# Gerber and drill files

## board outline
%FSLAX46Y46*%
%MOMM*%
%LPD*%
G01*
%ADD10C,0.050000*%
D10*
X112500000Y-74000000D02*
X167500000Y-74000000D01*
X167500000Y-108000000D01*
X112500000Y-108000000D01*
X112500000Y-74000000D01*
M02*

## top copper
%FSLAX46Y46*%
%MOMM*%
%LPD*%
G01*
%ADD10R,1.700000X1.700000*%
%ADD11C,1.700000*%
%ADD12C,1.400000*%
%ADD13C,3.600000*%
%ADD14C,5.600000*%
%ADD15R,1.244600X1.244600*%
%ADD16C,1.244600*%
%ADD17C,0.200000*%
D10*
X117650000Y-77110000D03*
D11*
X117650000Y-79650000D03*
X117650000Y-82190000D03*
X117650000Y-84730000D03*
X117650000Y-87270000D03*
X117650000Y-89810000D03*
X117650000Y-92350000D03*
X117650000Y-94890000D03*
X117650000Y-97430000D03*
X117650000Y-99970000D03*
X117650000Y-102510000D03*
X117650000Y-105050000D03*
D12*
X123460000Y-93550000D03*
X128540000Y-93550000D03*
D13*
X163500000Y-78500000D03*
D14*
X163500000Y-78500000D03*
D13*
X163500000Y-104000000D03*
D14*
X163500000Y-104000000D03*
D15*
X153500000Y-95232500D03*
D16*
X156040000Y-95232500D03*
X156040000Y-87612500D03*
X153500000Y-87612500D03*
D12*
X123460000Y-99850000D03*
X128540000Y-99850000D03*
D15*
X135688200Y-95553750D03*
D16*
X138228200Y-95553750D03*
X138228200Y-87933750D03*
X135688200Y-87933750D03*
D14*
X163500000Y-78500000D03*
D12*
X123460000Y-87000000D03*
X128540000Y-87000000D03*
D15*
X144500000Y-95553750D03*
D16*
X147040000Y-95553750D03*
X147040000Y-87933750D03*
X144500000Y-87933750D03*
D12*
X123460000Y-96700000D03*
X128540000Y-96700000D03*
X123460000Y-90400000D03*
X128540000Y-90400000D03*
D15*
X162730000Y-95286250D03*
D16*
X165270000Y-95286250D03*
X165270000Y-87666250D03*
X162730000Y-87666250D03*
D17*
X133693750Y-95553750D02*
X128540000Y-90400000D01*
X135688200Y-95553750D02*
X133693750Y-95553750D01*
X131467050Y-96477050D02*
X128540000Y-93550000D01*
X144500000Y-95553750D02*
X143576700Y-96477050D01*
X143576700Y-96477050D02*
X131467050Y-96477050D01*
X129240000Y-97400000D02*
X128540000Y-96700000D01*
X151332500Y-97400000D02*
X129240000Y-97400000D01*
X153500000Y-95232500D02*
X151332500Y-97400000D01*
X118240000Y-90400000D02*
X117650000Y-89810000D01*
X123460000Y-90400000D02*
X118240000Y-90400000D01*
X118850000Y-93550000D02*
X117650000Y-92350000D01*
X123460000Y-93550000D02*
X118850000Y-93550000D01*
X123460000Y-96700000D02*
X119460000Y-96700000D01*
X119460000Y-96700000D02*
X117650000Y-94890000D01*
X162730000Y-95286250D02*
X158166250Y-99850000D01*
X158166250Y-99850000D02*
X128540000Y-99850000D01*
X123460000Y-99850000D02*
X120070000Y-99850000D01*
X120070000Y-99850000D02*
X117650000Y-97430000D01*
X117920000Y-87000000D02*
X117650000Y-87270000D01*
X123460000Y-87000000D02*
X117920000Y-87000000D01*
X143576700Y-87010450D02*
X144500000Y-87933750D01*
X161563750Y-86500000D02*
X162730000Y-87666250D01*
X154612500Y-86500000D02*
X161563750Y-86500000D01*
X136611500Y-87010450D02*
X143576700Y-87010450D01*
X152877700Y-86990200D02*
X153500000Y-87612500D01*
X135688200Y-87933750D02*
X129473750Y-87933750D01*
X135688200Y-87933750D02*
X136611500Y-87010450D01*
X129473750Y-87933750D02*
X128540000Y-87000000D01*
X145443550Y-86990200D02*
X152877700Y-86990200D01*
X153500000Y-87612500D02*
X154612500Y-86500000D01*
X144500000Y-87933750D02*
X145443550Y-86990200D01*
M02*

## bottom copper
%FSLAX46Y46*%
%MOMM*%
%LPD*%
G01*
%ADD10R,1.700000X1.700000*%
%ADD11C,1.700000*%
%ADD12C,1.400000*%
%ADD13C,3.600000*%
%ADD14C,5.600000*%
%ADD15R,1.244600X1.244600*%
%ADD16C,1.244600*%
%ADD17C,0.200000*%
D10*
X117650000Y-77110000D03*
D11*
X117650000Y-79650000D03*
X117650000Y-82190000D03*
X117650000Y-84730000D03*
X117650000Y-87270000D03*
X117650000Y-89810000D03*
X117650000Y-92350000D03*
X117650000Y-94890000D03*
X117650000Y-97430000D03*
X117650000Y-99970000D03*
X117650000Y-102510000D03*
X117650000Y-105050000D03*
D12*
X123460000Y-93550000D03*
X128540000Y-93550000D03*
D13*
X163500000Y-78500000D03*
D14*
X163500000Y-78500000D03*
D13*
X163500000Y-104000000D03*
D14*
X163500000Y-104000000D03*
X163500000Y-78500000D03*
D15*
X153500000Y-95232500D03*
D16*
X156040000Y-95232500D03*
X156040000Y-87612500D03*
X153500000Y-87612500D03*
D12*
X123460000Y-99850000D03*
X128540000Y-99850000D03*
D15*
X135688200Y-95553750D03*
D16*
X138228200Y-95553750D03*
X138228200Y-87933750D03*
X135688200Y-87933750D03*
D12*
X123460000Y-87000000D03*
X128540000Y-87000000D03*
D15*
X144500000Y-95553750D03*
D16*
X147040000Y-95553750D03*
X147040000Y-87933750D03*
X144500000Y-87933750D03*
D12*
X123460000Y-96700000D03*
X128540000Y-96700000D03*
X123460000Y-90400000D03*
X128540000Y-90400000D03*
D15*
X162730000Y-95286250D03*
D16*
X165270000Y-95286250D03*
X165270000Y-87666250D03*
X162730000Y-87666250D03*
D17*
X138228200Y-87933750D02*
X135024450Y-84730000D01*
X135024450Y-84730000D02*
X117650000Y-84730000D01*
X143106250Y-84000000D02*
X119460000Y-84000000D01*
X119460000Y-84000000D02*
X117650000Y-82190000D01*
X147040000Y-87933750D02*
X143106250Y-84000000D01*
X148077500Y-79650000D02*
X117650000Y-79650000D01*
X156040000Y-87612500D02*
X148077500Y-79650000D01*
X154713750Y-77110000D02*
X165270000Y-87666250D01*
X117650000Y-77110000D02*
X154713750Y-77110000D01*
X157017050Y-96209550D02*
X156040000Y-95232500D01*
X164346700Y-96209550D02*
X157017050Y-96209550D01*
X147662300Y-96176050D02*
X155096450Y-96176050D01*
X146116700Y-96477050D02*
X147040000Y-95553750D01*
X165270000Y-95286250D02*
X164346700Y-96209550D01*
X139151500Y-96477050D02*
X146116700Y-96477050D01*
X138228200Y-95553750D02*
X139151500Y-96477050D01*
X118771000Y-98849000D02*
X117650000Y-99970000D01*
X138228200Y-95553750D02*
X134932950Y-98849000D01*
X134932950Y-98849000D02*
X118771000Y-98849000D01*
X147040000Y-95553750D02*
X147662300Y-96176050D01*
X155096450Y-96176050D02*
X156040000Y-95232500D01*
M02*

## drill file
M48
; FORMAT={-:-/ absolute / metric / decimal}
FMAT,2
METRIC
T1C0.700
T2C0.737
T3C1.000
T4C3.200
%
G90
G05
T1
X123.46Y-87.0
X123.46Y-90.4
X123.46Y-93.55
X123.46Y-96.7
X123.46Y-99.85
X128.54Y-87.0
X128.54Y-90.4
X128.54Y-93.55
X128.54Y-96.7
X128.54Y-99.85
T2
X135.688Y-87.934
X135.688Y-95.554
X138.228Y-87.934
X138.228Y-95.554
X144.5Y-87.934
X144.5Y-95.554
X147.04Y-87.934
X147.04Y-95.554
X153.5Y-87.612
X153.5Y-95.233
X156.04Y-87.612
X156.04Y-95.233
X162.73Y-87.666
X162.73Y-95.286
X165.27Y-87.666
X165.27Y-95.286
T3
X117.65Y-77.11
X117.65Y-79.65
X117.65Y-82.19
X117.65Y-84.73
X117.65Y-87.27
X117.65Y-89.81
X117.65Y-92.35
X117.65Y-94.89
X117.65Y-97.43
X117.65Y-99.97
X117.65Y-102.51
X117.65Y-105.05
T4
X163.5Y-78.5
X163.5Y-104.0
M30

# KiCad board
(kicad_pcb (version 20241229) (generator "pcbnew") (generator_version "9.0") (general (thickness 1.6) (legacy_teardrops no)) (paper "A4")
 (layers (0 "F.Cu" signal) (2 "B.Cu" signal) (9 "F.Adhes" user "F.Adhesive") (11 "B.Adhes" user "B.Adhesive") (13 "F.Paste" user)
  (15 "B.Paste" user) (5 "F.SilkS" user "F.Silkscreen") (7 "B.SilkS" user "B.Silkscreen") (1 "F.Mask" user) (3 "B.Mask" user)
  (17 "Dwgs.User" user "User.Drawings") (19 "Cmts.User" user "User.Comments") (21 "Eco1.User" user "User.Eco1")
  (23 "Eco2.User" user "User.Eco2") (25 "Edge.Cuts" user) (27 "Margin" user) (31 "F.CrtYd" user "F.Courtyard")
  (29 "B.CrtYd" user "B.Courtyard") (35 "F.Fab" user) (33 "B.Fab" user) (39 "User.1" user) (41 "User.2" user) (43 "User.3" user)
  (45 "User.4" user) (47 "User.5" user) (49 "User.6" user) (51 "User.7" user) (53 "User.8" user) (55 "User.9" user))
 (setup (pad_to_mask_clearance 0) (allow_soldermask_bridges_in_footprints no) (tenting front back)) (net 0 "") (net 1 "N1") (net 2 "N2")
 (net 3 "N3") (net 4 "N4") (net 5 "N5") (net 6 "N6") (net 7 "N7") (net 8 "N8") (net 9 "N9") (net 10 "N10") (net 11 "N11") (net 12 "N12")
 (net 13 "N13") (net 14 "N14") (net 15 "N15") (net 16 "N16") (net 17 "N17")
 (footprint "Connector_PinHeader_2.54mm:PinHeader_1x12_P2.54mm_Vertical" (layer "F.Cu") (at 117.65 77.11)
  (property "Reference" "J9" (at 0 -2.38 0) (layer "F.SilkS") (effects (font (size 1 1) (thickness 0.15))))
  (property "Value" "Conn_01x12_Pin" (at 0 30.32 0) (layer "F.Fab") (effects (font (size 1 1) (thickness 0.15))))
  (pad "1" thru_hole rect (at 0 0) (size 1.7 1.7) (drill 1) (layers "*.Cu" "*.Mask") (remove_unused_layers no) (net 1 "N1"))
  (pad "2" thru_hole circle (at 0 2.54) (size 1.7 1.7) (drill 1) (layers "*.Cu" "*.Mask") (remove_unused_layers no) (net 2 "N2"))
  (pad "3" thru_hole circle (at 0 5.08) (size 1.7 1.7) (drill 1) (layers "*.Cu" "*.Mask") (remove_unused_layers no) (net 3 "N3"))
  (pad "4" thru_hole circle (at 0 7.62) (size 1.7 1.7) (drill 1) (layers "*.Cu" "*.Mask") (remove_unused_layers no) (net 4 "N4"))
  (pad "5" thru_hole circle (at 0 10.16) (size 1.7 1.7) (drill 1) (layers "*.Cu" "*.Mask") (remove_unused_layers no) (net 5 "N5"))
  (pad "6" thru_hole circle (at 0 12.7) (size 1.7 1.7) (drill 1) (layers "*.Cu" "*.Mask") (remove_unused_layers no) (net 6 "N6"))
  (pad "7" thru_hole circle (at 0 15.24) (size 1.7 1.7) (drill 1) (layers "*.Cu" "*.Mask") (remove_unused_layers no) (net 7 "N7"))
  (pad "8" thru_hole circle (at 0 17.78) (size 1.7 1.7) (drill 1) (layers "*.Cu" "*.Mask") (remove_unused_layers no) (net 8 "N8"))
  (pad "9" thru_hole circle (at 0 20.32) (size 1.7 1.7) (drill 1) (layers "*.Cu" "*.Mask") (remove_unused_layers no) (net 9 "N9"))
  (pad "10" thru_hole circle (at 0 22.86) (size 1.7 1.7) (drill 1) (layers "*.Cu" "*.Mask") (remove_unused_layers no) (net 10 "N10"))
  (pad "11" thru_hole circle (at 0 25.4) (size 1.7 1.7) (drill 1) (layers "*.Cu" "*.Mask") (remove_unused_layers no) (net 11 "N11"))
  (pad "12" thru_hole circle (at 0 27.94) (size 1.7 1.7) (drill 1) (layers "*.Cu" "*.Mask") (remove_unused_layers no) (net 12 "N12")))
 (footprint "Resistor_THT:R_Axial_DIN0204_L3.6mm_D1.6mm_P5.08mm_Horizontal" (layer "F.Cu") (at 123.46 93.55)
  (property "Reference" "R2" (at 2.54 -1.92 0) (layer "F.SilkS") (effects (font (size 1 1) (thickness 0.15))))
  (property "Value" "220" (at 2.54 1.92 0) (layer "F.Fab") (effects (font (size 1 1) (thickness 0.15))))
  (pad "1" thru_hole circle (at 0 0) (size 1.4 1.4) (drill 0.7) (layers "*.Cu" "*.Mask") (remove_unused_layers no) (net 7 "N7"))
  (pad "2" thru_hole circle (at 5.08 0) (size 1.4 1.4) (drill 0.7) (layers "*.Cu" "*.Mask") (remove_unused_layers no) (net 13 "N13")))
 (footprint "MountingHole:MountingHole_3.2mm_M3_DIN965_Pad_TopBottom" (layer "F.Cu") (at 163.5 78.5)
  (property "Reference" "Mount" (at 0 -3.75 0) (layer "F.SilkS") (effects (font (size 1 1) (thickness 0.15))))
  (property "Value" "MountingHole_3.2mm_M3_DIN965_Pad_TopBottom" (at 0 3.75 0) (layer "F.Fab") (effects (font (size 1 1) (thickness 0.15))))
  (pad "1" thru_hole circle (at 0 0) (size 3.6 3.6) (drill 3.2) (layers "*.Cu" "*.Mask") (remove_unused_layers no) (zone_connect 2))
  (pad "1" connect circle (at 0 0) (size 5.6 5.6) (layers "F.Cu" "F.Mask") (zone_connect 2))
  (pad "1" connect circle (at 0 0) (size 5.6 5.6) (layers "B.Cu" "B.Mask") (zone_connect 2)))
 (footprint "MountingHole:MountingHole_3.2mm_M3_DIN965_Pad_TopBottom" (layer "F.Cu") (at 163.5 104)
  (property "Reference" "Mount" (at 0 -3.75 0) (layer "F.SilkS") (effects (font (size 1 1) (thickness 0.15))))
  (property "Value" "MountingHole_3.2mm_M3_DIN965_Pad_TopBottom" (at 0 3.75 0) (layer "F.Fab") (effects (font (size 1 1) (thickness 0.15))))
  (pad "1" thru_hole circle (at 0 0) (size 3.6 3.6) (drill 3.2) (layers "*.Cu" "*.Mask") (remove_unused_layers no) (zone_connect 2))
  (pad "1" connect circle (at 0 0) (size 5.6 5.6) (layers "F.Cu" "F.Mask") (zone_connect 2))
  (pad "1" connect circle (at 0 0) (size 5.6 5.6) (layers "B.Cu" "B.Mask") (zone_connect 2)))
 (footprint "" (layer "F.Cu") (at 163.5 78.5)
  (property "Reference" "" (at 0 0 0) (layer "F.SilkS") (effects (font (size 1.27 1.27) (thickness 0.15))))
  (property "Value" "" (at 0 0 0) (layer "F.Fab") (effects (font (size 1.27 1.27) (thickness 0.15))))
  (pad "1" connect circle (at 0 0) (size 5.6 5.6) (layers "B.Cu" "B.Mask") (zone_connect 2)))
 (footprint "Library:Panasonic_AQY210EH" (layer "F.Cu") (at 154.77 86.4225)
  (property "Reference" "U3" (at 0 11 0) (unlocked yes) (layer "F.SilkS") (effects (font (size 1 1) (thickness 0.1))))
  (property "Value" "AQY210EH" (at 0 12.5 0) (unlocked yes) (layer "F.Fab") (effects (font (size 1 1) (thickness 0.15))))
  (pad "1" thru_hole rect (at -1.27 8.81 90) (size 1.2446 1.2446) (drill 0.7366) (layers "*.Cu" "*.Mask") (remove_unused_layers no)
   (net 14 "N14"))
  (pad "2" thru_hole circle (at 1.27 8.81 90) (size 1.2446 1.2446) (drill 0.7366) (layers "*.Cu" "*.Mask") (remove_unused_layers no)
   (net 10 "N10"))
  (pad "3" thru_hole circle (at 1.27 1.19 90) (size 1.2446 1.2446) (drill 0.7366) (layers "*.Cu" "*.Mask") (remove_unused_layers no)
   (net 2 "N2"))
  (pad "4" thru_hole circle (at -1.27 1.19 90) (size 1.2446 1.2446) (drill 0.7366) (layers "*.Cu" "*.Mask") (remove_unused_layers no)
   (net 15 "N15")))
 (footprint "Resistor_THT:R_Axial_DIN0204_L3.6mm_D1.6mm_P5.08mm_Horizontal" (layer "F.Cu") (at 123.46 99.85)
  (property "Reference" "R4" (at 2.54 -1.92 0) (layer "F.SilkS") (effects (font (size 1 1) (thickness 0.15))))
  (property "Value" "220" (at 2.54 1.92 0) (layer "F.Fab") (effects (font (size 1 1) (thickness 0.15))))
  (pad "1" thru_hole circle (at 0 0) (size 1.4 1.4) (drill 0.7) (layers "*.Cu" "*.Mask") (remove_unused_layers no) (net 9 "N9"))
  (pad "2" thru_hole circle (at 5.08 0) (size 1.4 1.4) (drill 0.7) (layers "*.Cu" "*.Mask") (remove_unused_layers no) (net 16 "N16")))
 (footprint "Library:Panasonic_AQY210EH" (layer "F.Cu") (at 136.9582 86.74375)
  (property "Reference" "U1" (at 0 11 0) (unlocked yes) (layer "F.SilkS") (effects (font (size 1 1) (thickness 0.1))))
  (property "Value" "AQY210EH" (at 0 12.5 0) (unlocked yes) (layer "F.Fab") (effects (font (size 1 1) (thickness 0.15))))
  (pad "1" thru_hole rect (at -1.27 8.81 90) (size 1.2446 1.2446) (drill 0.7366) (layers "*.Cu" "*.Mask") (remove_unused_layers no)
   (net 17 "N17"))
  (pad "2" thru_hole circle (at 1.27 8.81 90) (size 1.2446 1.2446) (drill 0.7366) (layers "*.Cu" "*.Mask") (remove_unused_layers no)
   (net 10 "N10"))
  (pad "3" thru_hole circle (at 1.27 1.19 90) (size 1.2446 1.2446) (drill 0.7366) (layers "*.Cu" "*.Mask") (remove_unused_layers no)
   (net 4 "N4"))
  (pad "4" thru_hole circle (at -1.27 1.19 90) (size 1.2446 1.2446) (drill 0.7366) (layers "*.Cu" "*.Mask") (remove_unused_layers no)
   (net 15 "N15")))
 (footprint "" (layer "F.Cu") (at 163.5 78.5)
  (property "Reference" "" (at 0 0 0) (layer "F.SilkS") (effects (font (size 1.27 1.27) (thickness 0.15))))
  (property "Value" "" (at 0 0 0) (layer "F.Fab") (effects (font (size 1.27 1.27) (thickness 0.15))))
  (pad "1" connect circle (at 0 0) (size 5.6 5.6) (layers "F.Cu" "F.Mask") (zone_connect 2)))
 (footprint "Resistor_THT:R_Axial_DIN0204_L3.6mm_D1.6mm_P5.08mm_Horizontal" (layer "F.Cu") (at 123.46 87)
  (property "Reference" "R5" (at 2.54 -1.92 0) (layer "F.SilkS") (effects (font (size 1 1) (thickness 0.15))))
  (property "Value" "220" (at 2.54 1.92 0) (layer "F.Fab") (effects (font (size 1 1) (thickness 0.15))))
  (pad "1" thru_hole circle (at 0 0) (size 1.4 1.4) (drill 0.7) (layers "*.Cu" "*.Mask") (remove_unused_layers no) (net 5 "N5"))
  (pad "2" thru_hole circle (at 5.08 0) (size 1.4 1.4) (drill 0.7) (layers "*.Cu" "*.Mask") (remove_unused_layers no) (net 15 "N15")))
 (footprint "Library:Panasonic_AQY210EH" (layer "F.Cu") (at 145.77 86.74375)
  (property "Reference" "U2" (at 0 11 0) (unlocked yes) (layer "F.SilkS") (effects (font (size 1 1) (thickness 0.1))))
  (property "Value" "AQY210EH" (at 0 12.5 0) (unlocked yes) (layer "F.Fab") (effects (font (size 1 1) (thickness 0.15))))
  (pad "1" thru_hole rect (at -1.27 8.81 90) (size 1.2446 1.2446) (drill 0.7366) (layers "*.Cu" "*.Mask") (remove_unused_layers no)
   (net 13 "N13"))
  (pad "2" thru_hole circle (at 1.27 8.81 90) (size 1.2446 1.2446) (drill 0.7366) (layers "*.Cu" "*.Mask") (remove_unused_layers no)
   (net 10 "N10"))
  (pad "3" thru_hole circle (at 1.27 1.19 90) (size 1.2446 1.2446) (drill 0.7366) (layers "*.Cu" "*.Mask") (remove_unused_layers no)
   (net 3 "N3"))
  (pad "4" thru_hole circle (at -1.27 1.19 90) (size 1.2446 1.2446) (drill 0.7366) (layers "*.Cu" "*.Mask") (remove_unused_layers no)
   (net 15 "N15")))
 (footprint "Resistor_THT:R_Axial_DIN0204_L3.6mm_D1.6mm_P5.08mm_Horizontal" (layer "F.Cu") (at 123.46 96.7)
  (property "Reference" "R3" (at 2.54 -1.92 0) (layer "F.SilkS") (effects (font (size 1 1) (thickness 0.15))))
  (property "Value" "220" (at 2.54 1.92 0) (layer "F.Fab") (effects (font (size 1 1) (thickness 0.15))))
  (pad "1" thru_hole circle (at 0 0) (size 1.4 1.4) (drill 0.7) (layers "*.Cu" "*.Mask") (remove_unused_layers no) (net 8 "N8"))
  (pad "2" thru_hole circle (at 5.08 0) (size 1.4 1.4) (drill 0.7) (layers "*.Cu" "*.Mask") (remove_unused_layers no) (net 14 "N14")))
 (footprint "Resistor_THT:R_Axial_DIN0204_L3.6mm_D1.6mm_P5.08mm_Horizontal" (layer "F.Cu") (at 123.46 90.4)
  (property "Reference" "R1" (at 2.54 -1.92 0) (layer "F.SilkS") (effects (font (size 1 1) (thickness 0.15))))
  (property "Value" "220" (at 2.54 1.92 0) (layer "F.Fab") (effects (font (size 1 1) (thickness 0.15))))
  (pad "1" thru_hole circle (at 0 0) (size 1.4 1.4) (drill 0.7) (layers "*.Cu" "*.Mask") (remove_unused_layers no) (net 6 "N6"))
  (pad "2" thru_hole circle (at 5.08 0) (size 1.4 1.4) (drill 0.7) (layers "*.Cu" "*.Mask") (remove_unused_layers no) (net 17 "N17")))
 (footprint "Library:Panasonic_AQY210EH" (layer "F.Cu") (at 164 86.47625)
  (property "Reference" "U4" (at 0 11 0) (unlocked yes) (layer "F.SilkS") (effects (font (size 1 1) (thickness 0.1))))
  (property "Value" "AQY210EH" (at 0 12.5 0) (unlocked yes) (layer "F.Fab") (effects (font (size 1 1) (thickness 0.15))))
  (pad "1" thru_hole rect (at -1.27 8.81 90) (size 1.2446 1.2446) (drill 0.7366) (layers "*.Cu" "*.Mask") (remove_unused_layers no)
   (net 16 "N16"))
  (pad "2" thru_hole circle (at 1.27 8.81 90) (size 1.2446 1.2446) (drill 0.7366) (layers "*.Cu" "*.Mask") (remove_unused_layers no)
   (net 10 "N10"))
  (pad "3" thru_hole circle (at 1.27 1.19 90) (size 1.2446 1.2446) (drill 0.7366) (layers "*.Cu" "*.Mask") (remove_unused_layers no)
   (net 1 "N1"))
  (pad "4" thru_hole circle (at -1.27 1.19 90) (size 1.2446 1.2446) (drill 0.7366) (layers "*.Cu" "*.Mask") (remove_unused_layers no)
   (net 15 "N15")))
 (gr_rect (start 112.5 74) (end 167.5 108) (stroke (width 0.05) (type solid)) (fill no) (layer "Edge.Cuts"))
 (segment (start 133.69375 95.55375) (end 128.54 90.4) (width 0.2) (layer "F.Cu") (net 17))
 (segment (start 135.6882 95.55375) (end 133.69375 95.55375) (width 0.2) (layer "F.Cu") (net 17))
 (segment (start 131.46705 96.47705) (end 128.54 93.55) (width 0.2) (layer "F.Cu") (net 13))
 (segment (start 144.5 95.55375) (end 143.5767 96.47705) (width 0.2) (layer "F.Cu") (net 13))
 (segment (start 143.5767 96.47705) (end 131.46705 96.47705) (width 0.2) (layer "F.Cu") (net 13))
 (segment (start 129.24 97.4) (end 128.54 96.7) (width 0.2) (layer "F.Cu") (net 14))
 (segment (start 151.3325 97.4) (end 129.24 97.4) (width 0.2) (layer "F.Cu") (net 14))
 (segment (start 153.5 95.2325) (end 151.3325 97.4) (width 0.2) (layer "F.Cu") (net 14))
 (segment (start 118.24 90.4) (end 117.65 89.81) (width 0.2) (layer "F.Cu") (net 6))
 (segment (start 123.46 90.4) (end 118.24 90.4) (width 0.2) (layer "F.Cu") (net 6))
 (segment (start 118.85 93.55) (end 117.65 92.35) (width 0.2) (layer "F.Cu") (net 7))
 (segment (start 123.46 93.55) (end 118.85 93.55) (width 0.2) (layer "F.Cu") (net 7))
 (segment (start 123.46 96.7) (end 119.46 96.7) (width 0.2) (layer "F.Cu") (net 8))
 (segment (start 119.46 96.7) (end 117.65 94.89) (width 0.2) (layer "F.Cu") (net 8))
 (segment (start 162.73 95.28625) (end 158.16625 99.85) (width 0.2) (layer "F.Cu") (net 16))
 (segment (start 158.16625 99.85) (end 128.54 99.85) (width 0.2) (layer "F.Cu") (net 16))
 (segment (start 123.46 99.85) (end 120.07 99.85) (width 0.2) (layer "F.Cu") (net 9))
 (segment (start 120.07 99.85) (end 117.65 97.43) (width 0.2) (layer "F.Cu") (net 9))
 (segment (start 117.92 87) (end 117.65 87.27) (width 0.2) (layer "F.Cu") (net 5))
 (segment (start 123.46 87) (end 117.92 87) (width 0.2) (layer "F.Cu") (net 5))
 (segment (start 143.5767 87.01045) (end 144.5 87.93375) (width 0.2) (layer "F.Cu") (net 15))
 (segment (start 161.56375 86.5) (end 162.73 87.66625) (width 0.2) (layer "F.Cu") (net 15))
 (segment (start 154.6125 86.5) (end 161.56375 86.5) (width 0.2) (layer "F.Cu") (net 15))
 (segment (start 136.6115 87.01045) (end 143.5767 87.01045) (width 0.2) (layer "F.Cu") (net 15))
 (segment (start 152.8777 86.9902) (end 153.5 87.6125) (width 0.2) (layer "F.Cu") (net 15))
 (segment (start 135.6882 87.93375) (end 129.47375 87.93375) (width 0.2) (layer "F.Cu") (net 15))
 (segment (start 135.6882 87.93375) (end 136.6115 87.01045) (width 0.2) (layer "F.Cu") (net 15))
 (segment (start 129.47375 87.93375) (end 128.54 87) (width 0.2) (layer "F.Cu") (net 15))
 (segment (start 145.44355 86.9902) (end 152.8777 86.9902) (width 0.2) (layer "F.Cu") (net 15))
 (segment (start 153.5 87.6125) (end 154.6125 86.5) (width 0.2) (layer "F.Cu") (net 15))
 (segment (start 144.5 87.93375) (end 145.44355 86.9902) (width 0.2) (layer "F.Cu") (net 15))
 (segment (start 138.2282 87.93375) (end 135.02445 84.73) (width 0.2) (layer "B.Cu") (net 4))
 (segment (start 135.02445 84.73) (end 117.65 84.73) (width 0.2) (layer "B.Cu") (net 4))
 (segment (start 143.10625 84) (end 119.46 84) (width 0.2) (layer "B.Cu") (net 3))
 (segment (start 119.46 84) (end 117.65 82.19) (width 0.2) (layer "B.Cu") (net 3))
 (segment (start 147.04 87.93375) (end 143.10625 84) (width 0.2) (layer "B.Cu") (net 3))
 (segment (start 148.0775 79.65) (end 117.65 79.65) (width 0.2) (layer "B.Cu") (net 2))
 (segment (start 156.04 87.6125) (end 148.0775 79.65) (width 0.2) (layer "B.Cu") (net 2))
 (segment (start 154.71375 77.11) (end 165.27 87.66625) (width 0.2) (layer "B.Cu") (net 1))
 (segment (start 117.65 77.11) (end 154.71375 77.11) (width 0.2) (layer "B.Cu") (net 1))
 (segment (start 157.01705 96.20955) (end 156.04 95.2325) (width 0.2) (layer "B.Cu") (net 10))
 (segment (start 164.3467 96.20955) (end 157.01705 96.20955) (width 0.2) (layer "B.Cu") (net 10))
 (segment (start 147.6623 96.17605) (end 155.09645 96.17605) (width 0.2) (layer "B.Cu") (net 10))
 (segment (start 146.1167 96.47705) (end 147.04 95.55375) (width 0.2) (layer "B.Cu") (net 10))
 (segment (start 165.27 95.28625) (end 164.3467 96.20955) (width 0.2) (layer "B.Cu") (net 10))
 (segment (start 139.1515 96.47705) (end 146.1167 96.47705) (width 0.2) (layer "B.Cu") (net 10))
 (segment (start 138.2282 95.55375) (end 139.1515 96.47705) (width 0.2) (layer "B.Cu") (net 10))
 (segment (start 118.771 98.849) (end 117.65 99.97) (width 0.2) (layer "B.Cu") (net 10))
 (segment (start 138.2282 95.55375) (end 134.93295 98.849) (width 0.2) (layer "B.Cu") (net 10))
 (segment (start 134.93295 98.849) (end 118.771 98.849) (width 0.2) (layer "B.Cu") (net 10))
 (segment (start 147.04 95.55375) (end 147.6623 96.17605) (width 0.2) (layer "B.Cu") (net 10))
 (segment (start 155.09645 96.17605) (end 156.04 95.2325) (width 0.2) (layer "B.Cu") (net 10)))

